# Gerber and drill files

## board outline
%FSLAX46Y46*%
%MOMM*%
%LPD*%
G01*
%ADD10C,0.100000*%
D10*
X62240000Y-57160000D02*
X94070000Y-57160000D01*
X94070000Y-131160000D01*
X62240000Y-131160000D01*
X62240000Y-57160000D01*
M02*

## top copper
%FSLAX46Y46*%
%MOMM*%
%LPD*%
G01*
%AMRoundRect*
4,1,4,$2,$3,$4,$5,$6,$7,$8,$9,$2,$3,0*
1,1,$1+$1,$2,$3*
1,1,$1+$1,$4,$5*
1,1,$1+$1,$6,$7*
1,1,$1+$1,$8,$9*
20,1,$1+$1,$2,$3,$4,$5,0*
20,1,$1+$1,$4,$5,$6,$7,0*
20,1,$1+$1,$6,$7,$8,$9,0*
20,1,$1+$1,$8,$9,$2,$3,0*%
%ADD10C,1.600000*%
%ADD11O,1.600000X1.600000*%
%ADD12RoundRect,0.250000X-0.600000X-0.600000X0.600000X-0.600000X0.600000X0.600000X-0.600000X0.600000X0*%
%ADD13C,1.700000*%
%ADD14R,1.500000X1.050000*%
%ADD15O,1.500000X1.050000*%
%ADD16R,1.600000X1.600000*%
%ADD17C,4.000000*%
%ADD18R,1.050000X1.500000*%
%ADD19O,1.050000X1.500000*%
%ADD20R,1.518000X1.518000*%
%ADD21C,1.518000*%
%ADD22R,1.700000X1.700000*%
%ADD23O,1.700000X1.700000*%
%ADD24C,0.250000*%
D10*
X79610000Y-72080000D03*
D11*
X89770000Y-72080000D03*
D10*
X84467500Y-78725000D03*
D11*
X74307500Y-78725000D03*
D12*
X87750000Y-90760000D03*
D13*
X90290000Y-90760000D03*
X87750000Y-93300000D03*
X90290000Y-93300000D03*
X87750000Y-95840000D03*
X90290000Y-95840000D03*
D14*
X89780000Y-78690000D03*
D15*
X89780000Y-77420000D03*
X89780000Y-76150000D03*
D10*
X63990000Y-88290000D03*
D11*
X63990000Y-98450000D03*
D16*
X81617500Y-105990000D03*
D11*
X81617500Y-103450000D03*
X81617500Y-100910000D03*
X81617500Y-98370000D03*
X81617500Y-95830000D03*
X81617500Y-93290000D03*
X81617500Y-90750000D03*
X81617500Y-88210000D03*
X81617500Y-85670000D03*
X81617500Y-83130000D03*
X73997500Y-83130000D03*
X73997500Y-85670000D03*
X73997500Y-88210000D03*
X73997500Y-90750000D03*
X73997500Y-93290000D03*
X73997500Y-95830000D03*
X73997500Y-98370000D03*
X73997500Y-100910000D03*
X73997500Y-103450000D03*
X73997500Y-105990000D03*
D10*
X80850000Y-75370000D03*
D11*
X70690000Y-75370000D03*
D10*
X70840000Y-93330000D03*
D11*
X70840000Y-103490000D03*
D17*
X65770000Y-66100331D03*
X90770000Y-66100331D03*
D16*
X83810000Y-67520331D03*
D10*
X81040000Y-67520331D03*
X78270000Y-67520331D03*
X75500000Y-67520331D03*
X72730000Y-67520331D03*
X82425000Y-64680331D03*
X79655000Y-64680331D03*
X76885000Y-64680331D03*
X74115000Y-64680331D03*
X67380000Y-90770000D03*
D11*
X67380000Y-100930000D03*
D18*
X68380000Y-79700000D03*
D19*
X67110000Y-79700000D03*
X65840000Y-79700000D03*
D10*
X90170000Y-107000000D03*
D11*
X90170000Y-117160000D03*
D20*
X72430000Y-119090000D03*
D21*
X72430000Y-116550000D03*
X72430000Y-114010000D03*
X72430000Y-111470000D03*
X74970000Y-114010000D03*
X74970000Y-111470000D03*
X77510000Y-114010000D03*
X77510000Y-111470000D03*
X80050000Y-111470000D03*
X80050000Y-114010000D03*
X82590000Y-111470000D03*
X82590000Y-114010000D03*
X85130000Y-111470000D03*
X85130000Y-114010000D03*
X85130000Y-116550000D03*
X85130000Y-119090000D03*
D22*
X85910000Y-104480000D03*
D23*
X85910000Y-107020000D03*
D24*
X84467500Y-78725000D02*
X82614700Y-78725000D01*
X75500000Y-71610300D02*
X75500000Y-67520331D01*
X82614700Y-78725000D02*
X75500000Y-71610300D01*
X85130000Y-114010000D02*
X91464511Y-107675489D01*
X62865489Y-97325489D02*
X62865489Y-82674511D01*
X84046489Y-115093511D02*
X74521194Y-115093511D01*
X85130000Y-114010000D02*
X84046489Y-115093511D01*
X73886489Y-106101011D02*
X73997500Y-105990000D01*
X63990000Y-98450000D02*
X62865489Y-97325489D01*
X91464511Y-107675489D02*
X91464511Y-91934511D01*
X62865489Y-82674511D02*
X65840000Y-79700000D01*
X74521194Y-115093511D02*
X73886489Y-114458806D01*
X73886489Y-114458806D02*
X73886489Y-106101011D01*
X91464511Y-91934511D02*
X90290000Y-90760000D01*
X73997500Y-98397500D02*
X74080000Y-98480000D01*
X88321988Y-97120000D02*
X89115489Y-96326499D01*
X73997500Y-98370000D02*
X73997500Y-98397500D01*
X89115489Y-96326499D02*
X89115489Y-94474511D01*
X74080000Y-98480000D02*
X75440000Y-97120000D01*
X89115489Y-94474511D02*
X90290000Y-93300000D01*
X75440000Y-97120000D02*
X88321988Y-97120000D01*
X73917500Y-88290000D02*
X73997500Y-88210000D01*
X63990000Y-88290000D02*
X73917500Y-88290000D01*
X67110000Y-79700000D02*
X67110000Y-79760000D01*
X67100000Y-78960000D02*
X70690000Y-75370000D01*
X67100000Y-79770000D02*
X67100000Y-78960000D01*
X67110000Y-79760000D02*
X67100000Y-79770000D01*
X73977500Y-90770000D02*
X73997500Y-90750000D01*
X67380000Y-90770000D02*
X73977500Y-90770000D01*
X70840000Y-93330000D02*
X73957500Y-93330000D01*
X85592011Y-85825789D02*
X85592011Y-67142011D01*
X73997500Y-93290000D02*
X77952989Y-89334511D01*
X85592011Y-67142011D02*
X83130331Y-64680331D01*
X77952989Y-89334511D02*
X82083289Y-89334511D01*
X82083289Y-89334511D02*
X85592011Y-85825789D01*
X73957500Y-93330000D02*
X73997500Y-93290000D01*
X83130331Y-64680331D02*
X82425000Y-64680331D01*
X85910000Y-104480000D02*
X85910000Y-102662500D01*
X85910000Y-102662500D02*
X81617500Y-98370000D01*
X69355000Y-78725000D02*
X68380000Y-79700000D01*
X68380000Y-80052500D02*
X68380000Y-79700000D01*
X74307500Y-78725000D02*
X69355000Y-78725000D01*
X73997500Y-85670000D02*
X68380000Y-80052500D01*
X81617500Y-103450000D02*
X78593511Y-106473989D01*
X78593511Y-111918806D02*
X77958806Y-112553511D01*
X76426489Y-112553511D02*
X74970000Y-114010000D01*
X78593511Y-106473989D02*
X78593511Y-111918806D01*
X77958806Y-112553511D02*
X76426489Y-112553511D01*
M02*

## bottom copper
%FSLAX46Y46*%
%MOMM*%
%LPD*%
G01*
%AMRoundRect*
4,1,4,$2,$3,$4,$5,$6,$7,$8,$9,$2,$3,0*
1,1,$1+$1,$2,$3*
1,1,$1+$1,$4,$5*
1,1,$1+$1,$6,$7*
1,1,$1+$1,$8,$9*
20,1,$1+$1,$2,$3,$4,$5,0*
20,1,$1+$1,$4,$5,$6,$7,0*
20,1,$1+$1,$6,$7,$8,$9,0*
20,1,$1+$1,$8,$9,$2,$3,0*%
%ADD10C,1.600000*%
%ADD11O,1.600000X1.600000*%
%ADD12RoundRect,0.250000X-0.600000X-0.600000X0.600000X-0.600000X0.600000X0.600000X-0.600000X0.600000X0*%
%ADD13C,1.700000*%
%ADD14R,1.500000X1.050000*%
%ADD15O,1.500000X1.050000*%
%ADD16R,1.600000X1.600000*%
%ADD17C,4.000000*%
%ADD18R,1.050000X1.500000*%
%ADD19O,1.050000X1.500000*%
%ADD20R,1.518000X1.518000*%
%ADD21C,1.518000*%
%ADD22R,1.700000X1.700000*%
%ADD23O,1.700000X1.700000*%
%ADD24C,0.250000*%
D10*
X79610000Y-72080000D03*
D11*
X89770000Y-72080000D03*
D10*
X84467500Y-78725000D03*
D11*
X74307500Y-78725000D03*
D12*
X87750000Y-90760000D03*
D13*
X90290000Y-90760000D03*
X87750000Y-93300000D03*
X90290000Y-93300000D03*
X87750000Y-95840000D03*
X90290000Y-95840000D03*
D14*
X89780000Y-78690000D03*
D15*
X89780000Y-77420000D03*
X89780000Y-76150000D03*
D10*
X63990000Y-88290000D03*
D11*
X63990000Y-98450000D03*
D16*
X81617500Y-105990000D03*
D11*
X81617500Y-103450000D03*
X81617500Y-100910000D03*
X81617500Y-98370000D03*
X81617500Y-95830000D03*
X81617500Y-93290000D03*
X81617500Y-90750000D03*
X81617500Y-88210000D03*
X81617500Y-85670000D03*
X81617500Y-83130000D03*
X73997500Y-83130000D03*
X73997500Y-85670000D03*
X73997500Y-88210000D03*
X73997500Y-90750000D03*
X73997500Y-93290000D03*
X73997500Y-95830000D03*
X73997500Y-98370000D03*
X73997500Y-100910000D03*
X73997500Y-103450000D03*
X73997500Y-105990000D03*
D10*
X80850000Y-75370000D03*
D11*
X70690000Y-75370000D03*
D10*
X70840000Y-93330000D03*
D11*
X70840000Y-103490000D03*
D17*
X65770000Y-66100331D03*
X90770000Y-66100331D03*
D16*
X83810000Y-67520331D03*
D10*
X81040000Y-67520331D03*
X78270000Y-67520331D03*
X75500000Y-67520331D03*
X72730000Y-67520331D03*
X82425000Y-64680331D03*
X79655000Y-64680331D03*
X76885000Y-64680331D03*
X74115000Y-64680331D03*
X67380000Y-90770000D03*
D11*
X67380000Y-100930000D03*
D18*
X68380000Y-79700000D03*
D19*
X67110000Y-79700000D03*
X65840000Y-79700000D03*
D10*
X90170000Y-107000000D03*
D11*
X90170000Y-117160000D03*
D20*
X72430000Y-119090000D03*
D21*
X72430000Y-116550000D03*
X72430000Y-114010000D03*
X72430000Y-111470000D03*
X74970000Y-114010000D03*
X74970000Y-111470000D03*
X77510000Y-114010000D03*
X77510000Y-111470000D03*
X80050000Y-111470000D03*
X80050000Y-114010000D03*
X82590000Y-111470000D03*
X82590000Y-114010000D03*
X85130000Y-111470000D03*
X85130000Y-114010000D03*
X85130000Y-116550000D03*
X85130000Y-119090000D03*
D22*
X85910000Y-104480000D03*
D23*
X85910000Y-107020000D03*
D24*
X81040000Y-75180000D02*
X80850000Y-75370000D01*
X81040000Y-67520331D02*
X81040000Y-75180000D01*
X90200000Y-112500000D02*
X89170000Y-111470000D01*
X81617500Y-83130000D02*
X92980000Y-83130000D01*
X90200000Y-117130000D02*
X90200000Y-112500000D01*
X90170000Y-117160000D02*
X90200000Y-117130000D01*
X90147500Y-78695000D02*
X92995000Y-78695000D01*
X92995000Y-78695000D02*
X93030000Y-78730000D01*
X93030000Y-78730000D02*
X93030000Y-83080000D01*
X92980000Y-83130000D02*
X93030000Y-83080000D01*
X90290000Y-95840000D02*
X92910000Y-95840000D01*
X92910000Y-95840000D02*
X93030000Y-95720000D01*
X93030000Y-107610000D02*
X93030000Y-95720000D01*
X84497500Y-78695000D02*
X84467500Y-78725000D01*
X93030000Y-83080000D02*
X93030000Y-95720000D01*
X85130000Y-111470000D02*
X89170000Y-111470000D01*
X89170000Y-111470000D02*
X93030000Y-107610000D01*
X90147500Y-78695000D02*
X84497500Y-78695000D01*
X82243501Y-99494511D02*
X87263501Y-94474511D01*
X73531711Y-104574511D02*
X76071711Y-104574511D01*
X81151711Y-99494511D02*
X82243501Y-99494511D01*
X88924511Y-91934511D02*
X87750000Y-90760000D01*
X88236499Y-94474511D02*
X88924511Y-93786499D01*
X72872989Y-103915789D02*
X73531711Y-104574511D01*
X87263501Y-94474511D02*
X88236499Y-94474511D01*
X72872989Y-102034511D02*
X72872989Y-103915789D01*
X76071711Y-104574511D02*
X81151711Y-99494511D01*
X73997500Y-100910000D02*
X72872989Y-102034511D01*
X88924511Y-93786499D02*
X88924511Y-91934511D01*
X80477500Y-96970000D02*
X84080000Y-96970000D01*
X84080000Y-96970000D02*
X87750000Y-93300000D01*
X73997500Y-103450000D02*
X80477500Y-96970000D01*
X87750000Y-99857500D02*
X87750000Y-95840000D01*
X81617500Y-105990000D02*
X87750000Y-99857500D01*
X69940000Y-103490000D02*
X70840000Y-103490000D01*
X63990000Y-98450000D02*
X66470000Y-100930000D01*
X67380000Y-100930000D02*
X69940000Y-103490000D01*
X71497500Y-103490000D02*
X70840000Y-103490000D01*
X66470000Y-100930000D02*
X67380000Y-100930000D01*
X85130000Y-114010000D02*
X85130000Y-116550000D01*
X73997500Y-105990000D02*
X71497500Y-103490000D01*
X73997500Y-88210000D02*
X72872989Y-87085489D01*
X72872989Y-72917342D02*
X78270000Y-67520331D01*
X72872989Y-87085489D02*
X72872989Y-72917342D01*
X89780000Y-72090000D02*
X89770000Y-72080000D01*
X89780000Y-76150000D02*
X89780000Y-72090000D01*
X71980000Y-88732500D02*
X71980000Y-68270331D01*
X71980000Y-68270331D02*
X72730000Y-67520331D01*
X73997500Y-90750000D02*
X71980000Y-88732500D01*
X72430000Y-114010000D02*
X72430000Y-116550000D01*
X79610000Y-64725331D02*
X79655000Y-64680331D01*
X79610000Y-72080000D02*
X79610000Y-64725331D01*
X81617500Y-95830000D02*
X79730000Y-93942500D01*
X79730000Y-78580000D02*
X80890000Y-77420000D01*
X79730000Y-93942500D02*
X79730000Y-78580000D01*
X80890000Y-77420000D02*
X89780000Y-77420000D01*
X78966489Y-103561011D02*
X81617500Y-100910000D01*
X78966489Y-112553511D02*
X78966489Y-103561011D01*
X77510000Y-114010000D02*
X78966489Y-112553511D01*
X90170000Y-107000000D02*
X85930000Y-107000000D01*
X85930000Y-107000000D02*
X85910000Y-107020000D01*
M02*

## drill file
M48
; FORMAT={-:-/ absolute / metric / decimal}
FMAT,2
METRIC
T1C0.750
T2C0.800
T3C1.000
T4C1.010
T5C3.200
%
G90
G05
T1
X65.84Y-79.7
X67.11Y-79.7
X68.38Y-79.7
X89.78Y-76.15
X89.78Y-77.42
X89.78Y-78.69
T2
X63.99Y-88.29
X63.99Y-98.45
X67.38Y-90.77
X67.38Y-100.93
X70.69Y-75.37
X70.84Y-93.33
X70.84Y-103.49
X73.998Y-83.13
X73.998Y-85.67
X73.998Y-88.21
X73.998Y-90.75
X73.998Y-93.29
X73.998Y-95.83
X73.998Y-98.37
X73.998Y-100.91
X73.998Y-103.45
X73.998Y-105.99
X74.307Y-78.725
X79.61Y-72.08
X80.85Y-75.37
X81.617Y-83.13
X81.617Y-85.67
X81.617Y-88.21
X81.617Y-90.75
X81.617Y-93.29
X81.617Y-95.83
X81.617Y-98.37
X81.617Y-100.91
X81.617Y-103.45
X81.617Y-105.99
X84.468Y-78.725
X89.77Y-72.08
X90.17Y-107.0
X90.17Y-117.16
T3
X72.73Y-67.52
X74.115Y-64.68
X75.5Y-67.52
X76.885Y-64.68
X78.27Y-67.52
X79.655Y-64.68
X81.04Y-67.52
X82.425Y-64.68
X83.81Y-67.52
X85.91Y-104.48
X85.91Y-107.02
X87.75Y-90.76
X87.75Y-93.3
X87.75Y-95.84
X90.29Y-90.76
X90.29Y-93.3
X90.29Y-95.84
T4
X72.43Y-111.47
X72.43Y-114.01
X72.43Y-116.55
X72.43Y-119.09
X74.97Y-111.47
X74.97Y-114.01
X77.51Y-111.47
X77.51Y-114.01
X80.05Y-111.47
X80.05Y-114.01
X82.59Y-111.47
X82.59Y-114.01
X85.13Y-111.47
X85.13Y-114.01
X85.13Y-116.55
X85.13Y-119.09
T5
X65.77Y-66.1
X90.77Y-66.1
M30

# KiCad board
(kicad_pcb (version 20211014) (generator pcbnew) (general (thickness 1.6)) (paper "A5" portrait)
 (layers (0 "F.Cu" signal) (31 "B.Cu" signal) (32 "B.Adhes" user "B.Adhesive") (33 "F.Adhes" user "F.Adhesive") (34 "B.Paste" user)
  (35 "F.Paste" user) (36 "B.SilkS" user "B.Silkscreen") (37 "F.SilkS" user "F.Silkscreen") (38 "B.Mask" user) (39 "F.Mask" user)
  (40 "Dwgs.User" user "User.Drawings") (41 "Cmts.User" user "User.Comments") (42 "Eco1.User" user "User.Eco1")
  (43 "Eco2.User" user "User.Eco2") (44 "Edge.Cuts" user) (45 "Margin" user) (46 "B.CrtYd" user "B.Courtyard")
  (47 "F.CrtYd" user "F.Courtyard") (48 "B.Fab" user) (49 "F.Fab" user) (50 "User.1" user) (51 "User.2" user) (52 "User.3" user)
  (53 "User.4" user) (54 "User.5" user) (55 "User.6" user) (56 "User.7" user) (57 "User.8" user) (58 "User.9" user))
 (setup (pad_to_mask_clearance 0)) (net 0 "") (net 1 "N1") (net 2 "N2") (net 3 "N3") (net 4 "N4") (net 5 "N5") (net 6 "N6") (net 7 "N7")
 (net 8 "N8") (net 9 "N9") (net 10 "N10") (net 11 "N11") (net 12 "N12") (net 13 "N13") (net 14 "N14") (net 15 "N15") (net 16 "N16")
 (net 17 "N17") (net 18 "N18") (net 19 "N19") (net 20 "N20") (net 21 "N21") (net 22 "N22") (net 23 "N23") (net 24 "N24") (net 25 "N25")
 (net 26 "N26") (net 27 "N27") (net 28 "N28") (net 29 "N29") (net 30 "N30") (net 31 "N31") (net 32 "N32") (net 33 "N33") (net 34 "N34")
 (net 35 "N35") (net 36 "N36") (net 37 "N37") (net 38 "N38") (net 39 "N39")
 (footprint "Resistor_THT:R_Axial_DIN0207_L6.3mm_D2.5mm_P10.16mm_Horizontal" (layer "F.Cu") (at 79.61 72.08)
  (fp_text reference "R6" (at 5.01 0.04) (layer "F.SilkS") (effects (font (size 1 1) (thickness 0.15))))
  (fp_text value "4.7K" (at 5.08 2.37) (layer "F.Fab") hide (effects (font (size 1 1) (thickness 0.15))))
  (pad "1" thru_hole circle locked (at 0 0) (size 1.6 1.6) (drill 0.8) (layers *.Cu *.Mask) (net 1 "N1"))
  (pad "2" thru_hole oval locked (at 10.16 0) (size 1.6 1.6) (drill 0.8) (layers *.Cu *.Mask) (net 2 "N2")))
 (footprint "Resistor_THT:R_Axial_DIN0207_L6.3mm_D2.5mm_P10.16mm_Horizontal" (layer "F.Cu") (at 84.4675 78.725 180)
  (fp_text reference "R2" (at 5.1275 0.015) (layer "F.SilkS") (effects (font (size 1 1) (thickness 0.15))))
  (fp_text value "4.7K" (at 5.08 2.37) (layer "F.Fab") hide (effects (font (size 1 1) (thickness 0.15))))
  (pad "1" thru_hole circle locked (at 0 0 180) (size 1.6 1.6) (drill 0.8) (layers *.Cu *.Mask) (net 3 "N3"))
  (pad "2" thru_hole oval locked (at 10.16 0 180) (size 1.6 1.6) (drill 0.8) (layers *.Cu *.Mask) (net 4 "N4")))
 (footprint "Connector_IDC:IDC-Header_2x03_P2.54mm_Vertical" (layer "F.Cu") (at 87.75 90.76)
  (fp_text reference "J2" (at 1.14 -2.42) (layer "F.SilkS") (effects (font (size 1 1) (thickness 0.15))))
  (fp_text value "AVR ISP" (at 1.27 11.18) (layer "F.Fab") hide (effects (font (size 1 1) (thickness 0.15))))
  (pad "1" thru_hole roundrect locked (at 0 0) (size 1.7 1.7) (drill 1) (layers *.Cu *.Mask) (roundrect_rratio 0.1470588235) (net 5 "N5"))
  (pad "2" thru_hole circle locked (at 2.54 0) (size 1.7 1.7) (drill 1) (layers *.Cu *.Mask) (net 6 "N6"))
  (pad "3" thru_hole circle locked (at 0 2.54) (size 1.7 1.7) (drill 1) (layers *.Cu *.Mask) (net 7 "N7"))
  (pad "4" thru_hole circle locked (at 2.54 2.54) (size 1.7 1.7) (drill 1) (layers *.Cu *.Mask) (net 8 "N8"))
  (pad "5" thru_hole circle locked (at 0 5.08) (size 1.7 1.7) (drill 1) (layers *.Cu *.Mask) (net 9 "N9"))
  (pad "6" thru_hole circle locked (at 2.54 5.08) (size 1.7 1.7) (drill 1) (layers *.Cu *.Mask) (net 3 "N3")))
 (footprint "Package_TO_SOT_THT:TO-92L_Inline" (layer "F.Cu") (at 89.78 78.69 90)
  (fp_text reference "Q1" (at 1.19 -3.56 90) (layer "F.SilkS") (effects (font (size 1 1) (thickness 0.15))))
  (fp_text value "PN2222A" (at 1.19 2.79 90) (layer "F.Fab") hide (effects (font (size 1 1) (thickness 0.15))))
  (pad "1" thru_hole rect locked (at 0 0 90) (size 1.05 1.5) (drill 0.75) (layers *.Cu *.Mask) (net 3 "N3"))
  (pad "2" thru_hole oval locked (at 1.27 0 90) (size 1.05 1.5) (drill 0.75) (layers *.Cu *.Mask) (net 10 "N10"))
  (pad "3" thru_hole oval locked (at 2.54 0 90) (size 1.05 1.5) (drill 0.75) (layers *.Cu *.Mask) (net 2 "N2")))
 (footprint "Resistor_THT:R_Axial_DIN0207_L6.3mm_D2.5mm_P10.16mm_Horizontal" (layer "F.Cu") (at 63.99 88.29 -90)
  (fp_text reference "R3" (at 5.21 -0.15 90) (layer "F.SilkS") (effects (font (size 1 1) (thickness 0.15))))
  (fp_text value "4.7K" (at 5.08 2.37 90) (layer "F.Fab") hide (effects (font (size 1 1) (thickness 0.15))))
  (pad "1" thru_hole circle locked (at 0 0 270) (size 1.6 1.6) (drill 0.8) (layers *.Cu *.Mask) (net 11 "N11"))
  (pad "2" thru_hole oval locked (at 10.16 0 270) (size 1.6 1.6) (drill 0.8) (layers *.Cu *.Mask) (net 6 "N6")))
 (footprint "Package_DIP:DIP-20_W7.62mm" (layer "F.Cu") (at 81.6175 105.99 180)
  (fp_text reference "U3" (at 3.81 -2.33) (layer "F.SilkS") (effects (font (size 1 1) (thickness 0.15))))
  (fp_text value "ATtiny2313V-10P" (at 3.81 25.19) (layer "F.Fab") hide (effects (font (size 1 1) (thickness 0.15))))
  (pad "1" thru_hole rect locked (at 0 0 180) (size 1.6 1.6) (drill 0.8) (layers *.Cu *.Mask) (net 9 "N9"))
  (pad "2" thru_hole oval locked (at 0 2.54 180) (size 1.6 1.6) (drill 0.8) (layers *.Cu *.Mask) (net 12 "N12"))
  (pad "3" thru_hole oval locked (at 0 5.08 180) (size 1.6 1.6) (drill 0.8) (layers *.Cu *.Mask) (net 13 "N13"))
  (pad "4" thru_hole oval locked (at 0 7.62 180) (size 1.6 1.6) (drill 0.8) (layers *.Cu *.Mask) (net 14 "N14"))
  (pad "5" thru_hole oval locked (at 0 10.16 180) (size 1.6 1.6) (drill 0.8) (layers *.Cu *.Mask) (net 10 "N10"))
  (pad "6" thru_hole oval locked (at 0 12.7 180) (size 1.6 1.6) (drill 0.8) (layers *.Cu *.Mask) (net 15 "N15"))
  (pad "7" thru_hole oval locked (at 0 15.24 180) (size 1.6 1.6) (drill 0.8) (layers *.Cu *.Mask) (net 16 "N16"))
  (pad "8" thru_hole oval locked (at 0 17.78 180) (size 1.6 1.6) (drill 0.8) (layers *.Cu *.Mask) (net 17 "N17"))
  (pad "9" thru_hole oval locked (at 0 20.32 180) (size 1.6 1.6) (drill 0.8) (layers *.Cu *.Mask) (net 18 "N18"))
  (pad "10" thru_hole oval locked (at 0 22.86 180) (size 1.6 1.6) (drill 0.8) (layers *.Cu *.Mask) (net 3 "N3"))
  (pad "11" thru_hole oval locked (at 7.62 22.86 180) (size 1.6 1.6) (drill 0.8) (layers *.Cu *.Mask) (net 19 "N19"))
  (pad "12" thru_hole oval locked (at 7.62 20.32 180) (size 1.6 1.6) (drill 0.8) (layers *.Cu *.Mask) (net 4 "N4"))
  (pad "13" thru_hole oval locked (at 7.62 17.78 180) (size 1.6 1.6) (drill 0.8) (layers *.Cu *.Mask) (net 11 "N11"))
  (pad "14" thru_hole oval locked (at 7.62 15.24 180) (size 1.6 1.6) (drill 0.8) (layers *.Cu *.Mask) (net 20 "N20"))
  (pad "15" thru_hole oval locked (at 7.62 12.7 180) (size 1.6 1.6) (drill 0.8) (layers *.Cu *.Mask) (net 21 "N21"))
  (pad "16" thru_hole oval locked (at 7.62 10.16 180) (size 1.6 1.6) (drill 0.8) (layers *.Cu *.Mask) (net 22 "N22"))
  (pad "17" thru_hole oval locked (at 7.62 7.62 180) (size 1.6 1.6) (drill 0.8) (layers *.Cu *.Mask) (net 8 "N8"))
  (pad "18" thru_hole oval locked (at 7.62 5.08 180) (size 1.6 1.6) (drill 0.8) (layers *.Cu *.Mask) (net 5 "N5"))
  (pad "19" thru_hole oval locked (at 7.62 2.54 180) (size 1.6 1.6) (drill 0.8) (layers *.Cu *.Mask) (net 7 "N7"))
  (pad "20" thru_hole oval locked (at 7.62 0 180) (size 1.6 1.6) (drill 0.8) (layers *.Cu *.Mask) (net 6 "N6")))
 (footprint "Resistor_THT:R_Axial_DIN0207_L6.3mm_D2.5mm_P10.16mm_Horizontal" (layer "F.Cu") (at 80.85 75.37 180)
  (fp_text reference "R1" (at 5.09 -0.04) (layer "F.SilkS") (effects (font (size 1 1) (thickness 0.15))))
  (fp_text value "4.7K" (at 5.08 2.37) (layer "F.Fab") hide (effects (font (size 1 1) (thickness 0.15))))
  (pad "1" thru_hole circle locked (at 0 0 180) (size 1.6 1.6) (drill 0.8) (layers *.Cu *.Mask) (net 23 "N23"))
  (pad "2" thru_hole oval locked (at 10.16 0 180) (size 1.6 1.6) (drill 0.8) (layers *.Cu *.Mask) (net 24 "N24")))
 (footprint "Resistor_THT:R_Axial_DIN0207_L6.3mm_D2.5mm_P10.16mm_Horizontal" (layer "F.Cu") (at 70.84 93.33 -90)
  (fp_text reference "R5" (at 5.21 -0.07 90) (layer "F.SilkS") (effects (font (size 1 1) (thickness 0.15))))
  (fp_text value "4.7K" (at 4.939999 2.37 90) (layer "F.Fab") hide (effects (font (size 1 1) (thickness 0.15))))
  (pad "1" thru_hole circle locked (at 0 0 270) (size 1.6 1.6) (drill 0.8) (layers *.Cu *.Mask) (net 21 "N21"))
  (pad "2" thru_hole oval locked (at 10.16 0 270) (size 1.6 1.6) (drill 0.8) (layers *.Cu *.Mask) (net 6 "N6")))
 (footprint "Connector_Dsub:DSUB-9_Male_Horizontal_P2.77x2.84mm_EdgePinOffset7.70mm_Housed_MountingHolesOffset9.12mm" (layer "F.Cu")
  (at 83.81 67.520331 180)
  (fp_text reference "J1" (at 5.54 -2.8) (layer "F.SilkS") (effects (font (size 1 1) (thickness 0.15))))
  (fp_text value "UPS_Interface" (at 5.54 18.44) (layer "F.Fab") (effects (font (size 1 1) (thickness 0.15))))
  (pad "0" thru_hole circle locked (at 18.04 1.42 180) (size 4 4) (drill 3.2) (layers *.Cu *.Mask) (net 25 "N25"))
  (pad "0" thru_hole circle locked (at -6.96 1.42 180) (size 4 4) (drill 3.2) (layers *.Cu *.Mask) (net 25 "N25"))
  (pad "1" thru_hole rect locked (at 0 0 180) (size 1.6 1.6) (drill 1) (layers *.Cu *.Mask) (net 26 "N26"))
  (pad "2" thru_hole circle locked (at 2.77 0 180) (size 1.6 1.6) (drill 1) (layers *.Cu *.Mask) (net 23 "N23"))
  (pad "3" thru_hole circle locked (at 5.54 0 180) (size 1.6 1.6) (drill 1) (layers *.Cu *.Mask) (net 11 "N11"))
  (pad "4" thru_hole circle locked (at 8.31 0 180) (size 1.6 1.6) (drill 1) (layers *.Cu *.Mask) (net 3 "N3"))
  (pad "5" thru_hole circle locked (at 11.08 0 180) (size 1.6 1.6) (drill 1) (layers *.Cu *.Mask) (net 20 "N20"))
  (pad "6" thru_hole circle locked (at 1.385 2.84 180) (size 1.6 1.6) (drill 1) (layers *.Cu *.Mask) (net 21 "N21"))
  (pad "7" thru_hole circle locked (at 4.155 2.84 180) (size 1.6 1.6) (drill 1) (layers *.Cu *.Mask) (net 1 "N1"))
  (pad "8" thru_hole circle locked (at 6.925 2.84 180) (size 1.6 1.6) (drill 1) (layers *.Cu *.Mask) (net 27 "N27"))
  (pad "9" thru_hole circle locked (at 9.695 2.84 180) (size 1.6 1.6) (drill 1) (layers *.Cu *.Mask) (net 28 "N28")))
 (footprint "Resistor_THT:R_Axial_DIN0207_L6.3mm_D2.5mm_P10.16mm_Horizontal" (layer "F.Cu") (at 67.38 90.77 -90)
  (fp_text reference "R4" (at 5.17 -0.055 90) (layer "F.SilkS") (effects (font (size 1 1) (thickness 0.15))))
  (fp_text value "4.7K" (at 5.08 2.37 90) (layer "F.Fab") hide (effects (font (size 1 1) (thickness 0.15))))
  (pad "1" thru_hole circle locked (at 0 0 270) (size 1.6 1.6) (drill 0.8) (layers *.Cu *.Mask) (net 20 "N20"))
  (pad "2" thru_hole oval locked (at 10.16 0 270) (size 1.6 1.6) (drill 0.8) (layers *.Cu *.Mask) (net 6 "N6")))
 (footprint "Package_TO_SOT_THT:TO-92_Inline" (layer "F.Cu") (at 68.38 79.7 180)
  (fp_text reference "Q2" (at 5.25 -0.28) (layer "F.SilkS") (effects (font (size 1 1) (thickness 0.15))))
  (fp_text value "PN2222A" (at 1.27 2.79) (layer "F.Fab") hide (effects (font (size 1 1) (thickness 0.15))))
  (pad "1" thru_hole rect locked (at 0 0 180) (size 1.05 1.5) (drill 0.75) (layers *.Cu *.Mask) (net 4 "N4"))
  (pad "2" thru_hole oval locked (at 1.27 0 180) (size 1.05 1.5) (drill 0.75) (layers *.Cu *.Mask) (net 24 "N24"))
  (pad "3" thru_hole oval locked (at 2.54 0 180) (size 1.05 1.5) (drill 0.75) (layers *.Cu *.Mask) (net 6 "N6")))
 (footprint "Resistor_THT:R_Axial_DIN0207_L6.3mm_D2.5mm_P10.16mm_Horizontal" (layer "F.Cu") (at 90.17 107 -90) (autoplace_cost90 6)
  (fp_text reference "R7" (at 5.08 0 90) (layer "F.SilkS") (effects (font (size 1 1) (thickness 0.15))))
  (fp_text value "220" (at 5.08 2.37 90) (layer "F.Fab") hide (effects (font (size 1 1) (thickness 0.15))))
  (pad "1" thru_hole circle locked (at 0 0 270) (size 1.6 1.6) (drill 0.8) (layers *.Cu *.Mask) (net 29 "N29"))
  (pad "2" thru_hole oval locked (at 10.16 0 270) (size 1.6 1.6) (drill 0.8) (layers *.Cu *.Mask) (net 3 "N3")))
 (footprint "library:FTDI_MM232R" (layer "F.Cu") (at 78.78 120.34 90)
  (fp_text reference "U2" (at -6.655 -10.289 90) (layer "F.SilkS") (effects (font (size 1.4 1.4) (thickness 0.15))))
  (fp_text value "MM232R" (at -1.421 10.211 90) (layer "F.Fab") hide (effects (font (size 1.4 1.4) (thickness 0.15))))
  (pad "1" thru_hole rect locked (at 1.25 -6.35 90) (size 1.518 1.518) (drill 1.01) (layers *.Cu *.Mask) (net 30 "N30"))
  (pad "2" thru_hole circle locked (at 3.79 -6.35 90) (size 1.518 1.518) (drill 1.01) (layers *.Cu *.Mask) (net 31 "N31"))
  (pad "3" thru_hole circle locked (at 6.33 -6.35 90) (size 1.518 1.518) (drill 1.01) (layers *.Cu *.Mask) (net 31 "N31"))
  (pad "4" thru_hole circle locked (at 8.87 -6.35 90) (size 1.518 1.518) (drill 1.01) (layers *.Cu *.Mask) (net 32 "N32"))
  (pad "5" thru_hole circle locked (at 6.33 -3.81 90) (size 1.518 1.518) (drill 1.01) (layers *.Cu *.Mask) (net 12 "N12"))
  (pad "6" thru_hole circle locked (at 8.87 -3.81 90) (size 1.518 1.518) (drill 1.01) (layers *.Cu *.Mask) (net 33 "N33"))
  (pad "7" thru_hole circle locked (at 6.33 -1.27 90) (size 1.518 1.518) (drill 1.01) (layers *.Cu *.Mask) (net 13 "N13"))
  (pad "8" thru_hole circle locked (at 8.87 -1.27 90) (size 1.518 1.518) (drill 1.01) (layers *.Cu *.Mask) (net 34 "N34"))
  (pad "9" thru_hole circle locked (at 8.87 1.27 90) (size 1.518 1.518) (drill 1.01) (layers *.Cu *.Mask) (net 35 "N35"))
  (pad "10" thru_hole circle locked (at 6.33 1.27 90) (size 1.518 1.518) (drill 1.01) (layers *.Cu *.Mask) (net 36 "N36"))
  (pad "11" thru_hole circle locked (at 8.87 3.81 90) (size 1.518 1.518) (drill 1.01) (layers *.Cu *.Mask) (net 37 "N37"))
  (pad "12" thru_hole circle locked (at 6.33 3.81 90) (size 1.518 1.518) (drill 1.01) (layers *.Cu *.Mask) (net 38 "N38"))
  (pad "13" thru_hole circle locked (at 8.87 6.35 90) (size 1.518 1.518) (drill 1.01) (layers *.Cu *.Mask) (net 3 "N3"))
  (pad "14" thru_hole circle locked (at 6.33 6.35 90) (size 1.518 1.518) (drill 1.01) (layers *.Cu *.Mask) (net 6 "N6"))
  (pad "15" thru_hole circle locked (at 3.79 6.35 90) (size 1.518 1.518) (drill 1.01) (layers *.Cu *.Mask) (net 6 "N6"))
  (pad "16" thru_hole circle locked (at 1.25 6.35 90) (size 1.518 1.518) (drill 1.01) (layers *.Cu *.Mask) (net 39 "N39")))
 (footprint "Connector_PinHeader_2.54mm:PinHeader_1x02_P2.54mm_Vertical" (layer "F.Cu") (at 85.91 104.48)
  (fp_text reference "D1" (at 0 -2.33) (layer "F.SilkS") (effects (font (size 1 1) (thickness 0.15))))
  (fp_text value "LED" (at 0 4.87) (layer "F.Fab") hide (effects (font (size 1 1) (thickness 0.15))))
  (pad "1" thru_hole rect locked (at 0 0) (size 1.7 1.7) (drill 1) (layers *.Cu *.Mask) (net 14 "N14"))
  (pad "2" thru_hole oval locked (at 0 2.54) (size 1.7 1.7) (drill 1) (layers *.Cu *.Mask) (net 29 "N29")))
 (gr_rect (start 94.07 131.16) (end 62.24 57.16) (layer "Edge.Cuts") (width 0.1) (fill none))
 (segment (start 81.04 75.18) (end 80.85 75.37) (width 0.25) (layer "B.Cu") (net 23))
 (segment (start 81.04 67.520331) (end 81.04 75.18) (width 0.25) (layer "B.Cu") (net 23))
 (segment (start 84.4675 78.725) (end 82.6147 78.725) (width 0.25) (layer "F.Cu") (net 3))
 (segment (start 75.5 71.6103) (end 75.5 67.520331) (width 0.25) (layer "F.Cu") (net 3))
 (segment (start 82.6147 78.725) (end 75.5 71.6103) (width 0.25) (layer "F.Cu") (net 3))
 (segment (start 90.2 112.5) (end 89.17 111.47) (width 0.25) (layer "B.Cu") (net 3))
 (segment (start 81.6175 83.13) (end 92.98 83.13) (width 0.25) (layer "B.Cu") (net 3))
 (segment (start 90.2 117.13) (end 90.2 112.5) (width 0.25) (layer "B.Cu") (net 3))
 (segment (start 90.17 117.16) (end 90.2 117.13) (width 0.25) (layer "B.Cu") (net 3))
 (segment (start 90.1475 78.695) (end 92.995 78.695) (width 0.25) (layer "B.Cu") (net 3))
 (segment (start 92.995 78.695) (end 93.03 78.73) (width 0.25) (layer "B.Cu") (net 3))
 (segment (start 93.03 78.73) (end 93.03 83.08) (width 0.25) (layer "B.Cu") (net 3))
 (segment (start 92.98 83.13) (end 93.03 83.08) (width 0.25) (layer "B.Cu") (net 3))
 (segment (start 90.29 95.84) (end 92.91 95.84) (width 0.25) (layer "B.Cu") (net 3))
 (segment (start 92.91 95.84) (end 93.03 95.72) (width 0.25) (layer "B.Cu") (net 3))
 (segment (start 93.03 107.61) (end 93.03 95.72) (width 0.25) (layer "B.Cu") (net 3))
 (segment (start 84.4975 78.695) (end 84.4675 78.725) (width 0.25) (layer "B.Cu") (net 3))
 (segment (start 93.03 83.08) (end 93.03 95.72) (width 0.25) (layer "B.Cu") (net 3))
 (segment (start 85.13 111.47) (end 89.17 111.47) (width 0.25) (layer "B.Cu") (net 3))
 (segment (start 89.17 111.47) (end 93.03 107.61) (width 0.25) (layer "B.Cu") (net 3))
 (segment (start 90.1475 78.695) (end 84.4975 78.695) (width 0.25) (layer "B.Cu") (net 3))
 (segment (start 82.243501 99.494511) (end 87.263501 94.474511) (width 0.25) (layer "B.Cu") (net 5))
 (segment (start 73.531711 104.574511) (end 76.071711 104.574511) (width 0.25) (layer "B.Cu") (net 5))
 (segment (start 81.151711 99.494511) (end 82.243501 99.494511) (width 0.25) (layer "B.Cu") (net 5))
 (segment (start 88.924511 91.934511) (end 87.75 90.76) (width 0.25) (layer "B.Cu") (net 5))
 (segment (start 88.236499 94.474511) (end 88.924511 93.786499) (width 0.25) (layer "B.Cu") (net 5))
 (segment (start 72.872989 103.915789) (end 73.531711 104.574511) (width 0.25) (layer "B.Cu") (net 5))
 (segment (start 87.263501 94.474511) (end 88.236499 94.474511) (width 0.25) (layer "B.Cu") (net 5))
 (segment (start 72.872989 102.034511) (end 72.872989 103.915789) (width 0.25) (layer "B.Cu") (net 5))
 (segment (start 76.071711 104.574511) (end 81.151711 99.494511) (width 0.25) (layer "B.Cu") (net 5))
 (segment (start 73.9975 100.91) (end 72.872989 102.034511) (width 0.25) (layer "B.Cu") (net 5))
 (segment (start 88.924511 93.786499) (end 88.924511 91.934511) (width 0.25) (layer "B.Cu") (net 5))
 (segment (start 80.4775 96.97) (end 84.08 96.97) (width 0.25) (layer "B.Cu") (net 7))
 (segment (start 84.08 96.97) (end 87.75 93.3) (width 0.25) (layer "B.Cu") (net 7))
 (segment (start 73.9975 103.45) (end 80.4775 96.97) (width 0.25) (layer "B.Cu") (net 7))
 (segment (start 87.75 99.8575) (end 87.75 95.84) (width 0.25) (layer "B.Cu") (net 9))
 (segment (start 81.6175 105.99) (end 87.75 99.8575) (width 0.25) (layer "B.Cu") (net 9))
 (segment (start 85.13 114.01) (end 91.464511 107.675489) (width 0.25) (layer "F.Cu") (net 6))
 (segment (start 62.865489 97.325489) (end 62.865489 82.674511) (width 0.25) (layer "F.Cu") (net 6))
 (segment (start 84.046489 115.093511) (end 74.521194 115.093511) (width 0.25) (layer "F.Cu") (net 6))
 (segment (start 85.13 114.01) (end 84.046489 115.093511) (width 0.25) (layer "F.Cu") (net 6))
 (segment (start 73.886489 106.101011) (end 73.9975 105.99) (width 0.25) (layer "F.Cu") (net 6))
 (segment (start 63.99 98.45) (end 62.865489 97.325489) (width 0.25) (layer "F.Cu") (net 6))
 (segment (start 91.464511 107.675489) (end 91.464511 91.934511) (width 0.25) (layer "F.Cu") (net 6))
 (segment (start 62.865489 82.674511) (end 65.84 79.7) (width 0.25) (layer "F.Cu") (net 6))
 (segment (start 74.521194 115.093511) (end 73.886489 114.458806) (width 0.25) (layer "F.Cu") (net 6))
 (segment (start 73.886489 114.458806) (end 73.886489 106.101011) (width 0.25) (layer "F.Cu") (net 6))
 (segment (start 91.464511 91.934511) (end 90.29 90.76) (width 0.25) (layer "F.Cu") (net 6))
 (segment (start 69.94 103.49) (end 70.84 103.49) (width 0.25) (layer "B.Cu") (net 6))
 (segment (start 63.99 98.45) (end 66.47 100.93) (width 0.25) (layer "B.Cu") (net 6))
 (segment (start 67.38 100.93) (end 69.94 103.49) (width 0.25) (layer "B.Cu") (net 6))
 (segment (start 71.4975 103.49) (end 70.84 103.49) (width 0.25) (layer "B.Cu") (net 6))
 (segment (start 66.47 100.93) (end 67.38 100.93) (width 0.25) (layer "B.Cu") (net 6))
 (segment (start 85.13 114.01) (end 85.13 116.55) (width 0.25) (layer "B.Cu") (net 6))
 (segment (start 73.9975 105.99) (end 71.4975 103.49) (width 0.25) (layer "B.Cu") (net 6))
 (segment (start 73.9975 98.3975) (end 74.08 98.48) (width 0.25) (layer "F.Cu") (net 8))
 (segment (start 88.321988 97.12) (end 89.115489 96.326499) (width 0.25) (layer "F.Cu") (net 8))
 (segment (start 73.9975 98.37) (end 73.9975 98.3975) (width 0.25) (layer "F.Cu") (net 8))
 (segment (start 89.115489 96.326499) (end 89.115489 94.474511) (width 0.25) (layer "F.Cu") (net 8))
 (segment (start 74.08 98.48) (end 75.44 97.12) (width 0.25) (layer "F.Cu") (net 8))
 (segment (start 89.115489 94.474511) (end 90.29 93.3) (width 0.25) (layer "F.Cu") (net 8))
 (segment (start 75.44 97.12) (end 88.321988 97.12) (width 0.25) (layer "F.Cu") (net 8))
 (segment (start 73.9175 88.29) (end 73.9975 88.21) (width 0.25) (layer "F.Cu") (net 11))
 (segment (start 63.99 88.29) (end 73.9175 88.29) (width 0.25) (layer "F.Cu") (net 11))
 (segment (start 73.9975 88.21) (end 72.872989 87.085489) (width 0.25) (layer "B.Cu") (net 11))
 (segment (start 72.872989 72.917342) (end 78.27 67.520331) (width 0.25) (layer "B.Cu") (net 11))
 (segment (start 72.872989 87.085489) (end 72.872989 72.917342) (width 0.25) (layer "B.Cu") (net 11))
 (segment (start 89.78 72.09) (end 89.77 72.08) (width 0.25) (layer "B.Cu") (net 2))
 (segment (start 89.78 76.15) (end 89.78 72.09) (width 0.25) (layer "B.Cu") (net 2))
 (segment (start 67.11 79.7) (end 67.11 79.76) (width 0.25) (layer "F.Cu") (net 24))
 (segment (start 67.1 78.96) (end 70.69 75.37) (width 0.25) (layer "F.Cu") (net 24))
 (segment (start 67.1 79.77) (end 67.1 78.96) (width 0.25) (layer "F.Cu") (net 24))
 (segment (start 67.11 79.76) (end 67.1 79.77) (width 0.25) (layer "F.Cu") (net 24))
 (segment (start 73.9775 90.77) (end 73.9975 90.75) (width 0.25) (layer "F.Cu") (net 20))
 (segment (start 67.38 90.77) (end 73.9775 90.77) (width 0.25) (layer "F.Cu") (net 20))
 (segment (start 71.98 88.7325) (end 71.98 68.270331) (width 0.25) (layer "B.Cu") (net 20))
 (segment (start 71.98 68.270331) (end 72.73 67.520331) (width 0.25) (layer "B.Cu") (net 20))
 (segment (start 73.9975 90.75) (end 71.98 88.7325) (width 0.25) (layer "B.Cu") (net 20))
 (segment (start 72.43 114.01) (end 72.43 116.55) (width 0.25) (layer "B.Cu") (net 31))
 (segment (start 70.84 93.33) (end 73.9575 93.33) (width 0.25) (layer "F.Cu") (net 21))
 (segment (start 85.592011 85.825789) (end 85.592011 67.142011) (width 0.25) (layer "F.Cu") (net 21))
 (segment (start 73.9975 93.29) (end 77.952989 89.334511) (width 0.25) (layer "F.Cu") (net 21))
 (segment (start 85.592011 67.142011) (end 83.130331 64.680331) (width 0.25) (layer "F.Cu") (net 21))
 (segment (start 77.952989 89.334511) (end 82.083289 89.334511) (width 0.25) (layer "F.Cu") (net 21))
 (segment (start 82.083289 89.334511) (end 85.592011 85.825789) (width 0.25) (layer "F.Cu") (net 21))
 (segment (start 73.9575 93.33) (end 73.9975 93.29) (width 0.25) (layer "F.Cu") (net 21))
 (segment (start 83.130331 64.680331) (end 82.425 64.680331) (width 0.25) (layer "F.Cu") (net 21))
 (segment (start 79.61 64.725331) (end 79.655 64.680331) (width 0.25) (layer "B.Cu") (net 1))
 (segment (start 79.61 72.08) (end 79.61 64.725331) (width 0.25) (layer "B.Cu") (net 1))
 (segment (start 85.91 104.48) (end 85.91 102.6625) (width 0.25) (layer "F.Cu") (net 14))
 (segment (start 85.91 102.6625) (end 81.6175 98.37) (width 0.25) (layer "F.Cu") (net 14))
 (segment (start 81.6175 95.83) (end 79.73 93.9425) (width 0.25) (layer "B.Cu") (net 10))
 (segment (start 79.73 78.58) (end 80.89 77.42) (width 0.25) (layer "B.Cu") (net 10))
 (segment (start 79.73 93.9425) (end 79.73 78.58) (width 0.25) (layer "B.Cu") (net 10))
 (segment (start 80.89 77.42) (end 89.78 77.42) (width 0.25) (layer "B.Cu") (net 10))
 (segment (start 69.355 78.725) (end 68.38 79.7) (width 0.25) (layer "F.Cu") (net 4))
 (segment (start 68.38 80.0525) (end 68.38 79.7) (width 0.25) (layer "F.Cu") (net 4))
 (segment (start 74.3075 78.725) (end 69.355 78.725) (width 0.25) (layer "F.Cu") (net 4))
 (segment (start 73.9975 85.67) (end 68.38 80.0525) (width 0.25) (layer "F.Cu") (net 4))
 (segment (start 81.6175 103.45) (end 78.593511 106.473989) (width 0.25) (layer "F.Cu") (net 12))
 (segment (start 78.593511 111.918806) (end 77.958806 112.553511) (width 0.25) (layer "F.Cu") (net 12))
 (segment (start 76.426489 112.553511) (end 74.97 114.01) (width 0.25) (layer "F.Cu") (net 12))
 (segment (start 78.593511 106.473989) (end 78.593511 111.918806) (width 0.25) (layer "F.Cu") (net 12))
 (segment (start 77.958806 112.553511) (end 76.426489 112.553511) (width 0.25) (layer "F.Cu") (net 12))
 (segment (start 78.966489 103.561011) (end 81.6175 100.91) (width 0.25) (layer "B.Cu") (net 13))
 (segment (start 78.966489 112.553511) (end 78.966489 103.561011) (width 0.25) (layer "B.Cu") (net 13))
 (segment (start 77.51 114.01) (end 78.966489 112.553511) (width 0.25) (layer "B.Cu") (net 13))
 (segment (start 90.17 107) (end 85.93 107) (width 0.25) (layer "B.Cu") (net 29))
 (segment (start 85.93 107) (end 85.91 107.02) (width 0.25) (layer "B.Cu") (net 29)))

